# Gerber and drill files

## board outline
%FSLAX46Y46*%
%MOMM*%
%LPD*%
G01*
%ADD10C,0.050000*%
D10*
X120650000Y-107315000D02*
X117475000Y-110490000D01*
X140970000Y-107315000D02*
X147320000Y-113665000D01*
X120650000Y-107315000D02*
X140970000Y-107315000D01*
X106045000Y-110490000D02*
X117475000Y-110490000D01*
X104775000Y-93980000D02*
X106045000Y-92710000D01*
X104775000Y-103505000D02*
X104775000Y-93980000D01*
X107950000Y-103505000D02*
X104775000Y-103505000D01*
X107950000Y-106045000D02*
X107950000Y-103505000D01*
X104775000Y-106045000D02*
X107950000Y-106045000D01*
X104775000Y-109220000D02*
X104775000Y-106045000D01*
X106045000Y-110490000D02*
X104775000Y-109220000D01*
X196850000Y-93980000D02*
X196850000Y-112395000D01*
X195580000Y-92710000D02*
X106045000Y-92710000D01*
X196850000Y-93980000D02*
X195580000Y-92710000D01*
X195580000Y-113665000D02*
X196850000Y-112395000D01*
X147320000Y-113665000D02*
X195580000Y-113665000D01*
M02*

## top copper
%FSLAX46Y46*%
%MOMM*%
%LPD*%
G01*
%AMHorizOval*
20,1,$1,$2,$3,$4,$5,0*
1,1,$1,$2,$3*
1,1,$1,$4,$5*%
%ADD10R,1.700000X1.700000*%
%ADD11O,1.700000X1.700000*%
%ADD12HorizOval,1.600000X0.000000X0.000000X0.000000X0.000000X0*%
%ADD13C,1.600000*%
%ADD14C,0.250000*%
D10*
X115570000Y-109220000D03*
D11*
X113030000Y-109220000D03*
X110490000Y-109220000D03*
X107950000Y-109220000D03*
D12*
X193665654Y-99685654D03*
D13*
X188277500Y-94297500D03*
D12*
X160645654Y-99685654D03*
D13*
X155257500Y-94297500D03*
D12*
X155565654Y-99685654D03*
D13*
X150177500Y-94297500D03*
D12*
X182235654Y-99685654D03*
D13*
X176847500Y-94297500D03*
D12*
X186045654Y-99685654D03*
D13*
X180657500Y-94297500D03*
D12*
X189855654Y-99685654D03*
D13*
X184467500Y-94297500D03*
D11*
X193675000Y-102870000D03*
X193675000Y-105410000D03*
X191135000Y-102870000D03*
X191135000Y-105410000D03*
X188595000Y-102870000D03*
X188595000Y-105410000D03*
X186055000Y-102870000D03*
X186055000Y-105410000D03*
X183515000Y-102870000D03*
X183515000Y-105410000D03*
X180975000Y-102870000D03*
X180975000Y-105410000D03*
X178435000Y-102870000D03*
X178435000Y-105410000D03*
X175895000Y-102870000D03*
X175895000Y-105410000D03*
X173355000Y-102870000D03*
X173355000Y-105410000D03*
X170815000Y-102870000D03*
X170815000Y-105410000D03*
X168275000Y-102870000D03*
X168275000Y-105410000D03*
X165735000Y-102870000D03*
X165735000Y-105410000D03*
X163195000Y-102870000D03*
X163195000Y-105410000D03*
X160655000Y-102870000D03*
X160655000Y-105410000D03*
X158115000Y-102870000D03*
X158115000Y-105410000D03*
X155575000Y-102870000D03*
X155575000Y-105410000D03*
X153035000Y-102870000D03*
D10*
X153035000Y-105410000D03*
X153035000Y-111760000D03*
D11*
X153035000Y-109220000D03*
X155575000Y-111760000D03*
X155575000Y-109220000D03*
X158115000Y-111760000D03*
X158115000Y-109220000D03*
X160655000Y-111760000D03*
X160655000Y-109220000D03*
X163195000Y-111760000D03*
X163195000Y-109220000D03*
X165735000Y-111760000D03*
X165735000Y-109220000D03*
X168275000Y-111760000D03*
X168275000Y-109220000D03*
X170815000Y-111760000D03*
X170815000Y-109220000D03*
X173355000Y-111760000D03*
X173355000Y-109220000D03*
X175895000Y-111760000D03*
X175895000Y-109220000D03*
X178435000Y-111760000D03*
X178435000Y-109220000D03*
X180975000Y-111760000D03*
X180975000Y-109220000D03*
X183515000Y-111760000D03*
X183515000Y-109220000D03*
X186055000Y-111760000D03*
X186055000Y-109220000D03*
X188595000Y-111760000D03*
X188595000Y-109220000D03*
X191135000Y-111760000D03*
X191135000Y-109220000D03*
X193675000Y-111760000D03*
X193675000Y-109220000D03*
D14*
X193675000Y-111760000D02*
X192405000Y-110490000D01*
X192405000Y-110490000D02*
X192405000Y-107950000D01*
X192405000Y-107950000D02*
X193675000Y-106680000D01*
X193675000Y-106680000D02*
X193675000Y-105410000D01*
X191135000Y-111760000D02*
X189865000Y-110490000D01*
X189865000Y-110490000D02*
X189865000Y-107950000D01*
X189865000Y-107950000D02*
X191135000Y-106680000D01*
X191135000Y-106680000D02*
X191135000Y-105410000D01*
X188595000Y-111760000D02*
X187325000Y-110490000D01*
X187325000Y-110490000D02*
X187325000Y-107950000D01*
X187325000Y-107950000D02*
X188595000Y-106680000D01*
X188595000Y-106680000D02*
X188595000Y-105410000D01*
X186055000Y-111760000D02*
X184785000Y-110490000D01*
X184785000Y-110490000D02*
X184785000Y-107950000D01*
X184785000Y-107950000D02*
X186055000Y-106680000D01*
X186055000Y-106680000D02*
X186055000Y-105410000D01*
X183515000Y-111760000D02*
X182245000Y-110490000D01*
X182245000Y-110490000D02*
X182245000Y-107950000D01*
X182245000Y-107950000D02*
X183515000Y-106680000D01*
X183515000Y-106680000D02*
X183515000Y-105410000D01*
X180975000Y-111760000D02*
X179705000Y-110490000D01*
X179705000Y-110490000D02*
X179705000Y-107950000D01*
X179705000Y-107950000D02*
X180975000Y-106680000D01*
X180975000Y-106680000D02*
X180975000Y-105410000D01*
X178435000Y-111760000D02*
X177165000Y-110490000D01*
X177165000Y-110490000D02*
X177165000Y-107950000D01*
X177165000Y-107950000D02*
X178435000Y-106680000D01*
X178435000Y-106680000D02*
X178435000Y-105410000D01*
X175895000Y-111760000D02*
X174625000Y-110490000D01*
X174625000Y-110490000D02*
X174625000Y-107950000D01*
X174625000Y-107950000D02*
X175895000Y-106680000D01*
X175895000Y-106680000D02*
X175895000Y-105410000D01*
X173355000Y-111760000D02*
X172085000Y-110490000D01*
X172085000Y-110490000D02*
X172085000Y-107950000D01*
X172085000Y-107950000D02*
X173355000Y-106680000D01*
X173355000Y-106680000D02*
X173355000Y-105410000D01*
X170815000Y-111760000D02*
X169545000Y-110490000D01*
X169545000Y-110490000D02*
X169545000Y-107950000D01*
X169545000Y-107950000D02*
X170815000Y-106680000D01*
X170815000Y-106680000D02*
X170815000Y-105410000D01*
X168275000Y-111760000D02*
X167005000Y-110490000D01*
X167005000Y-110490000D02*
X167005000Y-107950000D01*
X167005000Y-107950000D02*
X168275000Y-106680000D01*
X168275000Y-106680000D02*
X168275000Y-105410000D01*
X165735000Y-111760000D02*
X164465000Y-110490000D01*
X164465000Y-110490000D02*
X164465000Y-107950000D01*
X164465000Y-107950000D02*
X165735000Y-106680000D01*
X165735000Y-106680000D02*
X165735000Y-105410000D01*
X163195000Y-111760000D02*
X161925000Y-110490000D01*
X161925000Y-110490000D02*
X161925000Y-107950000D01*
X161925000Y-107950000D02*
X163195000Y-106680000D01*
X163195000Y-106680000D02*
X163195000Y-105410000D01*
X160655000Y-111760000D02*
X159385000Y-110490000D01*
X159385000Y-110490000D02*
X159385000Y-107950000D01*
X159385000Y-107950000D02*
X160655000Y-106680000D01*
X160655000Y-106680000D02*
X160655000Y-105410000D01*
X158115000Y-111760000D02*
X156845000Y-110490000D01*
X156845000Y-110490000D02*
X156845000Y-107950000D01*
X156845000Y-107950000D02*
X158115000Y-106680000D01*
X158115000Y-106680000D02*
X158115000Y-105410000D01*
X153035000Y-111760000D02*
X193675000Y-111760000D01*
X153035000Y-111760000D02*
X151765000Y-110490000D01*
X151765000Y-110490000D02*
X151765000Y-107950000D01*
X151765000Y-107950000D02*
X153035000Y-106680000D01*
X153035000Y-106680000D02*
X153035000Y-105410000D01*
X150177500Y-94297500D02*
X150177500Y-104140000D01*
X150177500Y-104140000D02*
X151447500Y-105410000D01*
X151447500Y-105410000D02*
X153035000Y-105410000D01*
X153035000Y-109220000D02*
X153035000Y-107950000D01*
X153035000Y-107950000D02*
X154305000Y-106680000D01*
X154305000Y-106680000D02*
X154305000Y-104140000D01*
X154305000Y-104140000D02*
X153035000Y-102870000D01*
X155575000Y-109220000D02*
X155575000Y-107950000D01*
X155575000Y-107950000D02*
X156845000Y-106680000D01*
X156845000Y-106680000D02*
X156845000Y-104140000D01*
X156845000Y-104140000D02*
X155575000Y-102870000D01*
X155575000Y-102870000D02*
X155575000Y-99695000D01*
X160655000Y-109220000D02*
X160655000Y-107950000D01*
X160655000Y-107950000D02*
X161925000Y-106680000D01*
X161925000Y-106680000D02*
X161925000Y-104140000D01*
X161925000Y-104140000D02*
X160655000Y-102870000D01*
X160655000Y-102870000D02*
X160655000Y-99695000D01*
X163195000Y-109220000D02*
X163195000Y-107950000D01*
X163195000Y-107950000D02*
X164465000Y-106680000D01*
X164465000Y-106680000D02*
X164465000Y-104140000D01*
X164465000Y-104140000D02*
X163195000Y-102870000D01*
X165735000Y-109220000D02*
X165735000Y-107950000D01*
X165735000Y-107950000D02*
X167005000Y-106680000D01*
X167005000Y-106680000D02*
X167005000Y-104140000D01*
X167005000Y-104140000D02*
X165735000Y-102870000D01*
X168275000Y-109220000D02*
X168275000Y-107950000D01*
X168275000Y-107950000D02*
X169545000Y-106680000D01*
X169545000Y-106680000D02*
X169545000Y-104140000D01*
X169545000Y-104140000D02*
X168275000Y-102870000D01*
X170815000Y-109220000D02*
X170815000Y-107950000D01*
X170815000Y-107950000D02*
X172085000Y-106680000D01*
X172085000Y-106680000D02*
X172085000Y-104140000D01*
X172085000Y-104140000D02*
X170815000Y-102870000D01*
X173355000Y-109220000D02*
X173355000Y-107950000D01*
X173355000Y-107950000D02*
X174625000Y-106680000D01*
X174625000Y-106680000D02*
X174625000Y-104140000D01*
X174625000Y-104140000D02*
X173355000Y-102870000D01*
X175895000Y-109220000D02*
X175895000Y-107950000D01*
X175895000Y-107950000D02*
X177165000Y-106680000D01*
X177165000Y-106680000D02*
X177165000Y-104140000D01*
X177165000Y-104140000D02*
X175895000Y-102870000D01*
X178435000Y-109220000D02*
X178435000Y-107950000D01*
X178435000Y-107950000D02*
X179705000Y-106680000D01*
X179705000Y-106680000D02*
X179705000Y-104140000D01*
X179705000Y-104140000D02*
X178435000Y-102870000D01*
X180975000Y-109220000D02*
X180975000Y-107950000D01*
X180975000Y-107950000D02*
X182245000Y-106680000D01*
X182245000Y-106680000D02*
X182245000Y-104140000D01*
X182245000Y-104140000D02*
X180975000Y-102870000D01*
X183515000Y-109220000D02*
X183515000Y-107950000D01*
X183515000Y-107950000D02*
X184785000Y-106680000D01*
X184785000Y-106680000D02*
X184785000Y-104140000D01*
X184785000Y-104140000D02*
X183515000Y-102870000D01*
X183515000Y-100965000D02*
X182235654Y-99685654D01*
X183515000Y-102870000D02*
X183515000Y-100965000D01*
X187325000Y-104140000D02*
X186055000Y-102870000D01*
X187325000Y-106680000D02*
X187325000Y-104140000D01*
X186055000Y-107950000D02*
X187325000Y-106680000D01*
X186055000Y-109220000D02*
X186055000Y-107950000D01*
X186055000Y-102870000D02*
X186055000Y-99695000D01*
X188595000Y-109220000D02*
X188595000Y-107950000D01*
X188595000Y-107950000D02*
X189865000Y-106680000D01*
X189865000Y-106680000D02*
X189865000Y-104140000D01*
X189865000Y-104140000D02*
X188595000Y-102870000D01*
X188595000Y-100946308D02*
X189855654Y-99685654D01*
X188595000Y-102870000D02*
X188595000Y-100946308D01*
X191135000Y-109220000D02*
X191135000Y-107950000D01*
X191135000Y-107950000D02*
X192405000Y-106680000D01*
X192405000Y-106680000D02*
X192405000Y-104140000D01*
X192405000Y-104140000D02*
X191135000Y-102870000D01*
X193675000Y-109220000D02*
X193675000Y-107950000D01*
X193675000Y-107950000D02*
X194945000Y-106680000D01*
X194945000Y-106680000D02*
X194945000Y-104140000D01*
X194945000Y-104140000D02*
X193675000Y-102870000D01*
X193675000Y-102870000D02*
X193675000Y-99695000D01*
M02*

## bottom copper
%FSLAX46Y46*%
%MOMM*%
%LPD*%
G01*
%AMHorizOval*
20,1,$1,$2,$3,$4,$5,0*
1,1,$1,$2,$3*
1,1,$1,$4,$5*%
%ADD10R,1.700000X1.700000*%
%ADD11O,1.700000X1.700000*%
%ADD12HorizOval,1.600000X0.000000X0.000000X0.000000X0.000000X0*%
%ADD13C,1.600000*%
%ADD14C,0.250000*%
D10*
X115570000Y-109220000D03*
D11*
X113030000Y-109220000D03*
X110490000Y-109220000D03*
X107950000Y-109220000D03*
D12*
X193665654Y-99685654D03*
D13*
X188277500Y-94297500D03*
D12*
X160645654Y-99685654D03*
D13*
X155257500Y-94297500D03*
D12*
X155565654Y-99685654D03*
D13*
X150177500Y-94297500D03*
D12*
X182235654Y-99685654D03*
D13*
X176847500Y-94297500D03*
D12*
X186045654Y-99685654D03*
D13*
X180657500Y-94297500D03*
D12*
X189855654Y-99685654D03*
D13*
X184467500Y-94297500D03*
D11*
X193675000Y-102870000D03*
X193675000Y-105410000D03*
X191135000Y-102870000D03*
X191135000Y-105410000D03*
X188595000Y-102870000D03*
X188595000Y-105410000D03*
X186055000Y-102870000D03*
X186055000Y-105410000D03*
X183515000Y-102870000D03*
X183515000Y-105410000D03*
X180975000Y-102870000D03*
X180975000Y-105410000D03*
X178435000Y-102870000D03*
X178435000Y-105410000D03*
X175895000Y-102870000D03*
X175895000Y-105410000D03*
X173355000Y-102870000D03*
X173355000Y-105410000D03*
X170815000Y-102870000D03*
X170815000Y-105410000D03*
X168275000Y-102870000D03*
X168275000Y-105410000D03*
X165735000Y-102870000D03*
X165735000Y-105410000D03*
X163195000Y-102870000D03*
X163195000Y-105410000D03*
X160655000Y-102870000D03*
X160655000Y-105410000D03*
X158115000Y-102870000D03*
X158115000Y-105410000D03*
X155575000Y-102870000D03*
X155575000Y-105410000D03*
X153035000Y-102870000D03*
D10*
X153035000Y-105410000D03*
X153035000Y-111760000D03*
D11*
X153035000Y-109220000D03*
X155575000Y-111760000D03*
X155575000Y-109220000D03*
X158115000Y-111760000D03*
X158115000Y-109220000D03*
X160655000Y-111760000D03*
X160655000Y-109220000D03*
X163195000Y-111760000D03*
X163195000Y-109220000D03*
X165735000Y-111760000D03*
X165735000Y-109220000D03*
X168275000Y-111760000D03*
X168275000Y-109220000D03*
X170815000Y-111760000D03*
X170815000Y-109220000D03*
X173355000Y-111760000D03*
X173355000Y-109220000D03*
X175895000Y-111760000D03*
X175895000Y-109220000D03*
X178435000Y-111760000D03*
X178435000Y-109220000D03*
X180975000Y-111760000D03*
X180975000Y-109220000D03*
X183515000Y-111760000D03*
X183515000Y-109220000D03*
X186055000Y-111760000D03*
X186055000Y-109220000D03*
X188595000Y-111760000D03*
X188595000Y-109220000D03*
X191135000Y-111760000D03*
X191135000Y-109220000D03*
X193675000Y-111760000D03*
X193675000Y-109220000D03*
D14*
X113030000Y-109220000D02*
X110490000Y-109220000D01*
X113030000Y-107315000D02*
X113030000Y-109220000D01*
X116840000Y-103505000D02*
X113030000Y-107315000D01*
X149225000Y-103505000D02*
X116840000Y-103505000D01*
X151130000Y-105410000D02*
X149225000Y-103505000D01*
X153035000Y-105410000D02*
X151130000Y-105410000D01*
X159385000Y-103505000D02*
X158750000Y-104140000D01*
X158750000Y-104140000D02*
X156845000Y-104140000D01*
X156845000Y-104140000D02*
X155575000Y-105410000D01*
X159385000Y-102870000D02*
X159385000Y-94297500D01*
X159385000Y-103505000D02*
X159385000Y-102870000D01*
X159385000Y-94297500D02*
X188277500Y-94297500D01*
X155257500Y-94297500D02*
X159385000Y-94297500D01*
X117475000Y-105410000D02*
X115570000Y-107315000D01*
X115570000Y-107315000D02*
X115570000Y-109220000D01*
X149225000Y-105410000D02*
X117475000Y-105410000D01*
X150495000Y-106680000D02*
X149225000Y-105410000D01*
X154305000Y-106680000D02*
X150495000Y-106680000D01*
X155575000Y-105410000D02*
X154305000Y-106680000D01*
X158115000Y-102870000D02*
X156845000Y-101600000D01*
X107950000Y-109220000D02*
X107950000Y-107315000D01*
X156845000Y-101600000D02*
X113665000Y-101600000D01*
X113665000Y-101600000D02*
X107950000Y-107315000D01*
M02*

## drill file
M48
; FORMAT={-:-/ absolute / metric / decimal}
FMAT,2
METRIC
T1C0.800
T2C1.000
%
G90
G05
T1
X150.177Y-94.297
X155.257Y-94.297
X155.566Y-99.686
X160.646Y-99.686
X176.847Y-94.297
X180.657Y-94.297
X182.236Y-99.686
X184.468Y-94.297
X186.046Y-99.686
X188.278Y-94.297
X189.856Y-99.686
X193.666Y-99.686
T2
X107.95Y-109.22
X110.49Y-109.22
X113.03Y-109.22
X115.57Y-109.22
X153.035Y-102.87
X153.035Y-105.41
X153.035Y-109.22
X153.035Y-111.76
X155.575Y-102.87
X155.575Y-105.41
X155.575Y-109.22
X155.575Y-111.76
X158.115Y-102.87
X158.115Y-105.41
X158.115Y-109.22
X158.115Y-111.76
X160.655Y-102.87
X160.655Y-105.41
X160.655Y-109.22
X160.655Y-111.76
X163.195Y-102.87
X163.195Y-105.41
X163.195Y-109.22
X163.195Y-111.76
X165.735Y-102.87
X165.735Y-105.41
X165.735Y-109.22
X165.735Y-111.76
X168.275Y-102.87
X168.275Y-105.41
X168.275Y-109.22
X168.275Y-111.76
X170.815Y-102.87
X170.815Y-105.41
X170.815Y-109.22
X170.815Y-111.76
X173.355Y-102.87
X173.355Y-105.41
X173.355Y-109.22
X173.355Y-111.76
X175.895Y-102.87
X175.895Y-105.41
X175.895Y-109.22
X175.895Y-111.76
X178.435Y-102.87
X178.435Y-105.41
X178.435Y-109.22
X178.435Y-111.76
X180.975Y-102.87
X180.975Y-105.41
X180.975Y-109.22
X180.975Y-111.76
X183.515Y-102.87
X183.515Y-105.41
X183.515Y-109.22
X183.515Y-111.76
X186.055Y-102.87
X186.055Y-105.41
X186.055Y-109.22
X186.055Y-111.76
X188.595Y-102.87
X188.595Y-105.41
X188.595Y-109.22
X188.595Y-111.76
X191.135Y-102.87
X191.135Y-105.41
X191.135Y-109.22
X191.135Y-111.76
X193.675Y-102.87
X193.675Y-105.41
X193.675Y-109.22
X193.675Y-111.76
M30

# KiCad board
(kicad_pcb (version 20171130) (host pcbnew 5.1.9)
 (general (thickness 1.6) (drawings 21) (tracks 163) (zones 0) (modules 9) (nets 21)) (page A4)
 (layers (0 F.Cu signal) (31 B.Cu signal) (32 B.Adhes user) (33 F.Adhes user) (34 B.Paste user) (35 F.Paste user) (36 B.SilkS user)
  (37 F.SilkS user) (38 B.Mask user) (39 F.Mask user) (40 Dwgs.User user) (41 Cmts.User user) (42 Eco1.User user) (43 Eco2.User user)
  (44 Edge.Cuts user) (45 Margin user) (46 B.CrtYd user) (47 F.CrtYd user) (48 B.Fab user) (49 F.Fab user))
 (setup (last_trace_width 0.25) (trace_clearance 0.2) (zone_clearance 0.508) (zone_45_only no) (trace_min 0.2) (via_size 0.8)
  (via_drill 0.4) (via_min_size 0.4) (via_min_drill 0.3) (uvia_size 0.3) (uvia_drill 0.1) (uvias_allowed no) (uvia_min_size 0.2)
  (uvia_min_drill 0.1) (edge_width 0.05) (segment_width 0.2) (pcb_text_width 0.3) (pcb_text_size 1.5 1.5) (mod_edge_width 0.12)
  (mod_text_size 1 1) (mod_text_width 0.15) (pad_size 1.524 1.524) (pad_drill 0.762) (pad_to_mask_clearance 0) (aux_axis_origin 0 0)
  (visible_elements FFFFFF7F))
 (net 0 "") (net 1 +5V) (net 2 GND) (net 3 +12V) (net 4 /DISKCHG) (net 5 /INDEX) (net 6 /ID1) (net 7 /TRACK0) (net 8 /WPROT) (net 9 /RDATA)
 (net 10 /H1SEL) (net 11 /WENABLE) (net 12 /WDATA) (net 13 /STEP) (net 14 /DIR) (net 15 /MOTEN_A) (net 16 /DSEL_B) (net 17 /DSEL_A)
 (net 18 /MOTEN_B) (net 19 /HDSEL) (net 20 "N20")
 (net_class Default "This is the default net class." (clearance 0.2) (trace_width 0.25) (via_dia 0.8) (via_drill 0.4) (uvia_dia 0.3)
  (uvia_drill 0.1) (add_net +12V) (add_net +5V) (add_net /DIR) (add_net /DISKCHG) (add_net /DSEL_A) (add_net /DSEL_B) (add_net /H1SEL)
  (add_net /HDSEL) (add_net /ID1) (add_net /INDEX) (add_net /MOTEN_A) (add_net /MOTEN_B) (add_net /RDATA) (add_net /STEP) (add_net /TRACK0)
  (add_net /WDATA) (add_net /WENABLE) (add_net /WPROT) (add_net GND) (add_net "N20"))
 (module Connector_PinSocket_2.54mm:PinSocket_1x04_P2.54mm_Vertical (layer B.Cu) (at 115.57 109.22 90)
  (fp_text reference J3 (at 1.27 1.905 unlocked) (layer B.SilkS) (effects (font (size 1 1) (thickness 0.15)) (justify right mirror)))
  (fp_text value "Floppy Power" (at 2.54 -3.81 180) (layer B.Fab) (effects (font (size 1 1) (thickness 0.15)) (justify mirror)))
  (pad 1 thru_hole rect (at 0 0 90) (size 1.7 1.7) (drill 1) (layers *.Cu *.Mask) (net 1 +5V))
  (pad 2 thru_hole oval (at 0 -2.54 90) (size 1.7 1.7) (drill 1) (layers *.Cu *.Mask) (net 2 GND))
  (pad 3 thru_hole oval (at 0 -5.08 90) (size 1.7 1.7) (drill 1) (layers *.Cu *.Mask) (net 2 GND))
  (pad 4 thru_hole oval (at 0 -7.62 90) (size 1.7 1.7) (drill 1) (layers *.Cu *.Mask) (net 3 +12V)))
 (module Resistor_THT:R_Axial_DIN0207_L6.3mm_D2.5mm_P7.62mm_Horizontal (layer F.Cu) (at 188.2775 94.2975 315)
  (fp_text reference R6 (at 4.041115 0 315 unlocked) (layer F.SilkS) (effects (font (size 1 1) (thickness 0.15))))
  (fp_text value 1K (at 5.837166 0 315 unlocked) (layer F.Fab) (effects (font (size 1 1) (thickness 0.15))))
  (pad 2 thru_hole oval (at 7.62 0 315) (size 1.6 1.6) (drill 0.8) (layers *.Cu *.Mask) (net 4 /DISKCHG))
  (pad 1 thru_hole circle (at 0 0 315) (size 1.6 1.6) (drill 0.8) (layers *.Cu *.Mask) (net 1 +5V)))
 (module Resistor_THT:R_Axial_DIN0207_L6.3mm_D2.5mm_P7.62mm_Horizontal (layer F.Cu) (at 155.2575 94.2975 315)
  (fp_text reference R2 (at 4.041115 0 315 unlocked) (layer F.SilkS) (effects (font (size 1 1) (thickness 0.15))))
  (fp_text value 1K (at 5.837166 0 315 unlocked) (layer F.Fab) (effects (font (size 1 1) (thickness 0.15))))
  (pad 2 thru_hole oval (at 7.62 0 315) (size 1.6 1.6) (drill 0.8) (layers *.Cu *.Mask) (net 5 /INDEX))
  (pad 1 thru_hole circle (at 0 0 315) (size 1.6 1.6) (drill 0.8) (layers *.Cu *.Mask) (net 1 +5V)))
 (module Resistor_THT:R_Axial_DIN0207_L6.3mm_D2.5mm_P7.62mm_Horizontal (layer F.Cu) (at 150.1775 94.2975 315)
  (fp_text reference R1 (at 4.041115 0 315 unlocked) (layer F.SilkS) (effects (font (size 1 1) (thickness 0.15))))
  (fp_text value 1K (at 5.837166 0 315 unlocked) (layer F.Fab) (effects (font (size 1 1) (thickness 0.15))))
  (pad 2 thru_hole oval (at 7.62 0 315) (size 1.6 1.6) (drill 0.8) (layers *.Cu *.Mask) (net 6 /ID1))
  (pad 1 thru_hole circle (at 0 0 315) (size 1.6 1.6) (drill 0.8) (layers *.Cu *.Mask) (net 2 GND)))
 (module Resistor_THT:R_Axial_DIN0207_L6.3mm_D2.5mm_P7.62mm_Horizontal (layer F.Cu) (at 176.8475 94.2975 315)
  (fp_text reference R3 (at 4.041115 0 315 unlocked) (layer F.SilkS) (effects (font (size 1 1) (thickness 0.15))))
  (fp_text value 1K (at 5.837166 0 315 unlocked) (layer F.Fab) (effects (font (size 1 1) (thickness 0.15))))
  (pad 2 thru_hole oval (at 7.62 0 315) (size 1.6 1.6) (drill 0.8) (layers *.Cu *.Mask) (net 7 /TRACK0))
  (pad 1 thru_hole circle (at 0 0 315) (size 1.6 1.6) (drill 0.8) (layers *.Cu *.Mask) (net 1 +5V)))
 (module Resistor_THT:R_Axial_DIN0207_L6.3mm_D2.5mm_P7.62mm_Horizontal (layer F.Cu) (at 180.6575 94.2975 315)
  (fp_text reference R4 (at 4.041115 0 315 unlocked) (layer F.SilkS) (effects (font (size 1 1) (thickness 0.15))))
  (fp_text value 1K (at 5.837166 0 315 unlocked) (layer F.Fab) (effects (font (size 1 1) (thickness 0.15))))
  (pad 2 thru_hole oval (at 7.62 0 315) (size 1.6 1.6) (drill 0.8) (layers *.Cu *.Mask) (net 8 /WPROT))
  (pad 1 thru_hole circle (at 0 0 315) (size 1.6 1.6) (drill 0.8) (layers *.Cu *.Mask) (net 1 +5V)))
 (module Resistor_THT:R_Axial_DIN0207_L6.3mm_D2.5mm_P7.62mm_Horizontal (layer F.Cu) (at 184.4675 94.2975 315)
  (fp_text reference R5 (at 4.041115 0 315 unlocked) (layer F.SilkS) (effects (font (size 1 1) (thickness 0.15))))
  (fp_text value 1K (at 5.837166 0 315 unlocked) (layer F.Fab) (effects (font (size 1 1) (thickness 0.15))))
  (pad 2 thru_hole oval (at 7.62 0 315) (size 1.6 1.6) (drill 0.8) (layers *.Cu *.Mask) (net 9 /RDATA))
  (pad 1 thru_hole circle (at 0 0 315) (size 1.6 1.6) (drill 0.8) (layers *.Cu *.Mask) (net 1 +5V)))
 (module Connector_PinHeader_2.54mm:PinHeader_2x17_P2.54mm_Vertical (layer F.Cu) (at 153.035 105.41 90)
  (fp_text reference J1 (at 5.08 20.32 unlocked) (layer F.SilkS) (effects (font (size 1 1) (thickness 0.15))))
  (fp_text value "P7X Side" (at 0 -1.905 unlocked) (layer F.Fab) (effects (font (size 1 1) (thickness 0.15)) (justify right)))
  (pad 34 thru_hole oval (at 2.54 40.64 90) (size 1.7 1.7) (drill 1) (layers *.Cu *.Mask) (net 4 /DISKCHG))
  (pad 33 thru_hole oval (at 0 40.64 90) (size 1.7 1.7) (drill 1) (layers *.Cu *.Mask) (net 2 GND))
  (pad 32 thru_hole oval (at 2.54 38.1 90) (size 1.7 1.7) (drill 1) (layers *.Cu *.Mask) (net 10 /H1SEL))
  (pad 31 thru_hole oval (at 0 38.1 90) (size 1.7 1.7) (drill 1) (layers *.Cu *.Mask) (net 2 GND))
  (pad 30 thru_hole oval (at 2.54 35.56 90) (size 1.7 1.7) (drill 1) (layers *.Cu *.Mask) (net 9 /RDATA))
  (pad 29 thru_hole oval (at 0 35.56 90) (size 1.7 1.7) (drill 1) (layers *.Cu *.Mask) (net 2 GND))
  (pad 28 thru_hole oval (at 2.54 33.02 90) (size 1.7 1.7) (drill 1) (layers *.Cu *.Mask) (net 8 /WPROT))
  (pad 27 thru_hole oval (at 0 33.02 90) (size 1.7 1.7) (drill 1) (layers *.Cu *.Mask) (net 2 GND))
  (pad 26 thru_hole oval (at 2.54 30.48 90) (size 1.7 1.7) (drill 1) (layers *.Cu *.Mask) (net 7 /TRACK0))
  (pad 25 thru_hole oval (at 0 30.48 90) (size 1.7 1.7) (drill 1) (layers *.Cu *.Mask) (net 2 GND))
  (pad 24 thru_hole oval (at 2.54 27.94 90) (size 1.7 1.7) (drill 1) (layers *.Cu *.Mask) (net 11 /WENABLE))
  (pad 23 thru_hole oval (at 0 27.94 90) (size 1.7 1.7) (drill 1) (layers *.Cu *.Mask) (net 2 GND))
  (pad 22 thru_hole oval (at 2.54 25.4 90) (size 1.7 1.7) (drill 1) (layers *.Cu *.Mask) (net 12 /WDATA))
  (pad 21 thru_hole oval (at 0 25.4 90) (size 1.7 1.7) (drill 1) (layers *.Cu *.Mask) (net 2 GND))
  (pad 20 thru_hole oval (at 2.54 22.86 90) (size 1.7 1.7) (drill 1) (layers *.Cu *.Mask) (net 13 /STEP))
  (pad 19 thru_hole oval (at 0 22.86 90) (size 1.7 1.7) (drill 1) (layers *.Cu *.Mask) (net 2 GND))
  (pad 18 thru_hole oval (at 2.54 20.32 90) (size 1.7 1.7) (drill 1) (layers *.Cu *.Mask) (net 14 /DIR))
  (pad 17 thru_hole oval (at 0 20.32 90) (size 1.7 1.7) (drill 1) (layers *.Cu *.Mask) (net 2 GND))
  (pad 16 thru_hole oval (at 2.54 17.78 90) (size 1.7 1.7) (drill 1) (layers *.Cu *.Mask) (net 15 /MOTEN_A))
  (pad 15 thru_hole oval (at 0 17.78 90) (size 1.7 1.7) (drill 1) (layers *.Cu *.Mask) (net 2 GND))
  (pad 14 thru_hole oval (at 2.54 15.24 90) (size 1.7 1.7) (drill 1) (layers *.Cu *.Mask) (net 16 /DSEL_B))
  (pad 13 thru_hole oval (at 0 15.24 90) (size 1.7 1.7) (drill 1) (layers *.Cu *.Mask) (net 2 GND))
  (pad 12 thru_hole oval (at 2.54 12.7 90) (size 1.7 1.7) (drill 1) (layers *.Cu *.Mask) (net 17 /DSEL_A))
  (pad 11 thru_hole oval (at 0 12.7 90) (size 1.7 1.7) (drill 1) (layers *.Cu *.Mask) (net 2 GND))
  (pad 10 thru_hole oval (at 2.54 10.16 90) (size 1.7 1.7) (drill 1) (layers *.Cu *.Mask) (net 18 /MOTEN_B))
  (pad 9 thru_hole oval (at 0 10.16 90) (size 1.7 1.7) (drill 1) (layers *.Cu *.Mask) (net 2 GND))
  (pad 8 thru_hole oval (at 2.54 7.62 90) (size 1.7 1.7) (drill 1) (layers *.Cu *.Mask) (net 5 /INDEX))
  (pad 7 thru_hole oval (at 0 7.62 90) (size 1.7 1.7) (drill 1) (layers *.Cu *.Mask) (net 2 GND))
  (pad 6 thru_hole oval (at 2.54 5.08 90) (size 1.7 1.7) (drill 1) (layers *.Cu *.Mask) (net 3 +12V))
  (pad 5 thru_hole oval (at 0 5.08 90) (size 1.7 1.7) (drill 1) (layers *.Cu *.Mask) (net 2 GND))
  (pad 4 thru_hole oval (at 2.54 2.54 90) (size 1.7 1.7) (drill 1) (layers *.Cu *.Mask) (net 6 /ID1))
  (pad 3 thru_hole oval (at 0 2.54 90) (size 1.7 1.7) (drill 1) (layers *.Cu *.Mask) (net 1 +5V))
  (pad 2 thru_hole oval (at 2.54 0 90) (size 1.7 1.7) (drill 1) (layers *.Cu *.Mask) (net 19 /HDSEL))
  (pad 1 thru_hole rect (at 0 0 90) (size 1.7 1.7) (drill 1) (layers *.Cu *.Mask) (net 2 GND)))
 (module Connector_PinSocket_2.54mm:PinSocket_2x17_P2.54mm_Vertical (layer B.Cu) (at 153.035 111.76 270)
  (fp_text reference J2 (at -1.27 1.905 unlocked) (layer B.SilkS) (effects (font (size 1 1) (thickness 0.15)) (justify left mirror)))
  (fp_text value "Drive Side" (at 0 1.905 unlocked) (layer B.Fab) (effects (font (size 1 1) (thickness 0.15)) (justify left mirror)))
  (pad 1 thru_hole rect (at 0 0 270) (size 1.7 1.7) (drill 1) (layers *.Cu *.Mask) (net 2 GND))
  (pad 2 thru_hole oval (at -2.54 0 270) (size 1.7 1.7) (drill 1) (layers *.Cu *.Mask) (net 19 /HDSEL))
  (pad 3 thru_hole oval (at 0 -2.54 270) (size 1.7 1.7) (drill 1) (layers *.Cu *.Mask) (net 2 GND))
  (pad 4 thru_hole oval (at -2.54 -2.54 270) (size 1.7 1.7) (drill 1) (layers *.Cu *.Mask) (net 6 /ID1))
  (pad 5 thru_hole oval (at 0 -5.08 270) (size 1.7 1.7) (drill 1) (layers *.Cu *.Mask) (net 2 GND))
  (pad 6 thru_hole oval (at -2.54 -5.08 270) (size 1.7 1.7) (drill 1) (layers *.Cu *.Mask) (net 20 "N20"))
  (pad 7 thru_hole oval (at 0 -7.62 270) (size 1.7 1.7) (drill 1) (layers *.Cu *.Mask) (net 2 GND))
  (pad 8 thru_hole oval (at -2.54 -7.62 270) (size 1.7 1.7) (drill 1) (layers *.Cu *.Mask) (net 5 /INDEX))
  (pad 9 thru_hole oval (at 0 -10.16 270) (size 1.7 1.7) (drill 1) (layers *.Cu *.Mask) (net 2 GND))
  (pad 10 thru_hole oval (at -2.54 -10.16 270) (size 1.7 1.7) (drill 1) (layers *.Cu *.Mask) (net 18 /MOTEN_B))
  (pad 11 thru_hole oval (at 0 -12.7 270) (size 1.7 1.7) (drill 1) (layers *.Cu *.Mask) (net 2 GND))
  (pad 12 thru_hole oval (at -2.54 -12.7 270) (size 1.7 1.7) (drill 1) (layers *.Cu *.Mask) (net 17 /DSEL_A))
  (pad 13 thru_hole oval (at 0 -15.24 270) (size 1.7 1.7) (drill 1) (layers *.Cu *.Mask) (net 2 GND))
  (pad 14 thru_hole oval (at -2.54 -15.24 270) (size 1.7 1.7) (drill 1) (layers *.Cu *.Mask) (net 16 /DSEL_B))
  (pad 15 thru_hole oval (at 0 -17.78 270) (size 1.7 1.7) (drill 1) (layers *.Cu *.Mask) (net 2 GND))
  (pad 16 thru_hole oval (at -2.54 -17.78 270) (size 1.7 1.7) (drill 1) (layers *.Cu *.Mask) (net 15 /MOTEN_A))
  (pad 17 thru_hole oval (at 0 -20.32 270) (size 1.7 1.7) (drill 1) (layers *.Cu *.Mask) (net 2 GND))
  (pad 18 thru_hole oval (at -2.54 -20.32 270) (size 1.7 1.7) (drill 1) (layers *.Cu *.Mask) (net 14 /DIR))
  (pad 19 thru_hole oval (at 0 -22.86 270) (size 1.7 1.7) (drill 1) (layers *.Cu *.Mask) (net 2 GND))
  (pad 20 thru_hole oval (at -2.54 -22.86 270) (size 1.7 1.7) (drill 1) (layers *.Cu *.Mask) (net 13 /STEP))
  (pad 21 thru_hole oval (at 0 -25.4 270) (size 1.7 1.7) (drill 1) (layers *.Cu *.Mask) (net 2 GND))
  (pad 22 thru_hole oval (at -2.54 -25.4 270) (size 1.7 1.7) (drill 1) (layers *.Cu *.Mask) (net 12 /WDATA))
  (pad 23 thru_hole oval (at 0 -27.94 270) (size 1.7 1.7) (drill 1) (layers *.Cu *.Mask) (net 2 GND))
  (pad 24 thru_hole oval (at -2.54 -27.94 270) (size 1.7 1.7) (drill 1) (layers *.Cu *.Mask) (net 11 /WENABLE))
  (pad 25 thru_hole oval (at 0 -30.48 270) (size 1.7 1.7) (drill 1) (layers *.Cu *.Mask) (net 2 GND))
  (pad 26 thru_hole oval (at -2.54 -30.48 270) (size 1.7 1.7) (drill 1) (layers *.Cu *.Mask) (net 7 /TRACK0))
  (pad 27 thru_hole oval (at 0 -33.02 270) (size 1.7 1.7) (drill 1) (layers *.Cu *.Mask) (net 2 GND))
  (pad 28 thru_hole oval (at -2.54 -33.02 270) (size 1.7 1.7) (drill 1) (layers *.Cu *.Mask) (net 8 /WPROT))
  (pad 29 thru_hole oval (at 0 -35.56 270) (size 1.7 1.7) (drill 1) (layers *.Cu *.Mask) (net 2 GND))
  (pad 30 thru_hole oval (at -2.54 -35.56 270) (size 1.7 1.7) (drill 1) (layers *.Cu *.Mask) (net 9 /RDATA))
  (pad 31 thru_hole oval (at 0 -38.1 270) (size 1.7 1.7) (drill 1) (layers *.Cu *.Mask) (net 2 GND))
  (pad 32 thru_hole oval (at -2.54 -38.1 270) (size 1.7 1.7) (drill 1) (layers *.Cu *.Mask) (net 10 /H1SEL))
  (pad 33 thru_hole oval (at 0 -40.64 270) (size 1.7 1.7) (drill 1) (layers *.Cu *.Mask) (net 2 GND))
  (pad 34 thru_hole oval (at -2.54 -40.64 270) (size 1.7 1.7) (drill 1) (layers *.Cu *.Mask) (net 4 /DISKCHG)))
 (gr_line (start 120.65 107.315) (end 117.475 110.49) (layer Edge.Cuts) (width 0.05))
 (gr_line (start 140.97 107.315) (end 147.32 113.665) (layer Edge.Cuts) (width 0.05))
 (gr_line (start 120.65 107.315) (end 140.97 107.315) (layer Edge.Cuts) (width 0.05))
 (gr_line (start 106.045 110.49) (end 117.475 110.49) (layer Edge.Cuts) (width 0.05))
 (gr_line (start 104.775 93.98) (end 106.045 92.71) (layer Edge.Cuts) (width 0.05))
 (gr_line (start 104.775 103.505) (end 104.775 93.98) (layer Edge.Cuts) (width 0.05))
 (gr_line (start 107.95 103.505) (end 104.775 103.505) (layer Edge.Cuts) (width 0.05))
 (gr_line (start 107.95 106.045) (end 107.95 103.505) (layer Edge.Cuts) (width 0.05))
 (gr_line (start 104.775 106.045) (end 107.95 106.045) (layer Edge.Cuts) (width 0.05))
 (gr_line (start 104.775 109.22) (end 104.775 106.045) (layer Edge.Cuts) (width 0.05))
 (gr_line (start 106.045 110.49) (end 104.775 109.22) (layer Edge.Cuts) (width 0.05))
 (gr_line (start 196.85 93.98) (end 196.85 112.395) (layer Edge.Cuts) (width 0.05))
 (gr_line (start 195.58 92.71) (end 106.045 92.71) (layer Edge.Cuts) (width 0.05))
 (gr_line (start 196.85 93.98) (end 195.58 92.71) (layer Edge.Cuts) (width 0.05))
 (gr_line (start 195.58 113.665) (end 196.85 112.395) (layer Edge.Cuts) (width 0.05))
 (gr_line (start 147.32 113.665) (end 195.58 113.665) (layer Edge.Cuts) (width 0.05))
 (segment (start 193.675 111.76) (end 192.405 110.49) (width 0.25) (layer F.Cu) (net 2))
 (segment (start 192.405 110.49) (end 192.405 107.95) (width 0.25) (layer F.Cu) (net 2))
 (segment (start 192.405 107.95) (end 193.675 106.68) (width 0.25) (layer F.Cu) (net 2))
 (segment (start 193.675 106.68) (end 193.675 105.41) (width 0.25) (layer F.Cu) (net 2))
 (segment (start 191.135 111.76) (end 189.865 110.49) (width 0.25) (layer F.Cu) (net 2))
 (segment (start 189.865 110.49) (end 189.865 107.95) (width 0.25) (layer F.Cu) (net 2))
 (segment (start 189.865 107.95) (end 191.135 106.68) (width 0.25) (layer F.Cu) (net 2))
 (segment (start 191.135 106.68) (end 191.135 105.41) (width 0.25) (layer F.Cu) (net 2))
 (segment (start 188.595 111.76) (end 187.325 110.49) (width 0.25) (layer F.Cu) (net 2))
 (segment (start 187.325 110.49) (end 187.325 107.95) (width 0.25) (layer F.Cu) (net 2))
 (segment (start 187.325 107.95) (end 188.595 106.68) (width 0.25) (layer F.Cu) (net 2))
 (segment (start 188.595 106.68) (end 188.595 105.41) (width 0.25) (layer F.Cu) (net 2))
 (segment (start 186.055 111.76) (end 184.785 110.49) (width 0.25) (layer F.Cu) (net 2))
 (segment (start 184.785 110.49) (end 184.785 107.95) (width 0.25) (layer F.Cu) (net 2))
 (segment (start 184.785 107.95) (end 186.055 106.68) (width 0.25) (layer F.Cu) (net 2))
 (segment (start 186.055 106.68) (end 186.055 105.41) (width 0.25) (layer F.Cu) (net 2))
 (segment (start 183.515 111.76) (end 182.245 110.49) (width 0.25) (layer F.Cu) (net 2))
 (segment (start 182.245 110.49) (end 182.245 107.95) (width 0.25) (layer F.Cu) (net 2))
 (segment (start 182.245 107.95) (end 183.515 106.68) (width 0.25) (layer F.Cu) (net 2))
 (segment (start 183.515 106.68) (end 183.515 105.41) (width 0.25) (layer F.Cu) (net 2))
 (segment (start 180.975 111.76) (end 179.705 110.49) (width 0.25) (layer F.Cu) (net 2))
 (segment (start 179.705 110.49) (end 179.705 107.95) (width 0.25) (layer F.Cu) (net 2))
 (segment (start 179.705 107.95) (end 180.975 106.68) (width 0.25) (layer F.Cu) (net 2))
 (segment (start 180.975 106.68) (end 180.975 105.41) (width 0.25) (layer F.Cu) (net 2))
 (segment (start 178.435 111.76) (end 177.165 110.49) (width 0.25) (layer F.Cu) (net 2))
 (segment (start 177.165 110.49) (end 177.165 107.95) (width 0.25) (layer F.Cu) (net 2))
 (segment (start 177.165 107.95) (end 178.435 106.68) (width 0.25) (layer F.Cu) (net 2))
 (segment (start 178.435 106.68) (end 178.435 105.41) (width 0.25) (layer F.Cu) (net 2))
 (segment (start 175.895 111.76) (end 174.625 110.49) (width 0.25) (layer F.Cu) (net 2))
 (segment (start 174.625 110.49) (end 174.625 107.95) (width 0.25) (layer F.Cu) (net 2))
 (segment (start 174.625 107.95) (end 175.895 106.68) (width 0.25) (layer F.Cu) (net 2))
 (segment (start 175.895 106.68) (end 175.895 105.41) (width 0.25) (layer F.Cu) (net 2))
 (segment (start 173.355 111.76) (end 172.085 110.49) (width 0.25) (layer F.Cu) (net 2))
 (segment (start 172.085 110.49) (end 172.085 107.95) (width 0.25) (layer F.Cu) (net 2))
 (segment (start 172.085 107.95) (end 173.355 106.68) (width 0.25) (layer F.Cu) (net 2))
 (segment (start 173.355 106.68) (end 173.355 105.41) (width 0.25) (layer F.Cu) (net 2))
 (segment (start 170.815 111.76) (end 169.545 110.49) (width 0.25) (layer F.Cu) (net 2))
 (segment (start 169.545 110.49) (end 169.545 107.95) (width 0.25) (layer F.Cu) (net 2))
 (segment (start 169.545 107.95) (end 170.815 106.68) (width 0.25) (layer F.Cu) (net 2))
 (segment (start 170.815 106.68) (end 170.815 105.41) (width 0.25) (layer F.Cu) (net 2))
 (segment (start 168.275 111.76) (end 167.005 110.49) (width 0.25) (layer F.Cu) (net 2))
 (segment (start 167.005 110.49) (end 167.005 107.95) (width 0.25) (layer F.Cu) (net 2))
 (segment (start 167.005 107.95) (end 168.275 106.68) (width 0.25) (layer F.Cu) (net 2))
 (segment (start 168.275 106.68) (end 168.275 105.41) (width 0.25) (layer F.Cu) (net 2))
 (segment (start 165.735 111.76) (end 164.465 110.49) (width 0.25) (layer F.Cu) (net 2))
 (segment (start 164.465 110.49) (end 164.465 107.95) (width 0.25) (layer F.Cu) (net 2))
 (segment (start 164.465 107.95) (end 165.735 106.68) (width 0.25) (layer F.Cu) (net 2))
 (segment (start 165.735 106.68) (end 165.735 105.41) (width 0.25) (layer F.Cu) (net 2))
 (segment (start 163.195 111.76) (end 161.925 110.49) (width 0.25) (layer F.Cu) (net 2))
 (segment (start 161.925 110.49) (end 161.925 107.95) (width 0.25) (layer F.Cu) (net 2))
 (segment (start 161.925 107.95) (end 163.195 106.68) (width 0.25) (layer F.Cu) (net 2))
 (segment (start 163.195 106.68) (end 163.195 105.41) (width 0.25) (layer F.Cu) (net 2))
 (segment (start 160.655 111.76) (end 159.385 110.49) (width 0.25) (layer F.Cu) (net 2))
 (segment (start 159.385 110.49) (end 159.385 107.95) (width 0.25) (layer F.Cu) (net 2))
 (segment (start 159.385 107.95) (end 160.655 106.68) (width 0.25) (layer F.Cu) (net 2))
 (segment (start 160.655 106.68) (end 160.655 105.41) (width 0.25) (layer F.Cu) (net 2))
 (segment (start 158.115 111.76) (end 156.845 110.49) (width 0.25) (layer F.Cu) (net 2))
 (segment (start 156.845 110.49) (end 156.845 107.95) (width 0.25) (layer F.Cu) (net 2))
 (segment (start 156.845 107.95) (end 158.115 106.68) (width 0.25) (layer F.Cu) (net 2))
 (segment (start 158.115 106.68) (end 158.115 105.41) (width 0.25) (layer F.Cu) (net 2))
 (segment (start 153.035 111.76) (end 193.675 111.76) (width 0.25) (layer F.Cu) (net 2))
 (segment (start 153.035 111.76) (end 151.765 110.49) (width 0.25) (layer F.Cu) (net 2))
 (segment (start 151.765 110.49) (end 151.765 107.95) (width 0.25) (layer F.Cu) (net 2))
 (segment (start 151.765 107.95) (end 153.035 106.68) (width 0.25) (layer F.Cu) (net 2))
 (segment (start 153.035 106.68) (end 153.035 105.41) (width 0.25) (layer F.Cu) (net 2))
 (segment (start 113.03 109.22) (end 110.49 109.22) (width 0.25) (layer B.Cu) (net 2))
 (segment (start 150.1775 94.2975) (end 150.1775 104.14) (width 0.25) (layer F.Cu) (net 2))
 (segment (start 150.1775 104.14) (end 151.4475 105.41) (width 0.25) (layer F.Cu) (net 2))
 (segment (start 151.4475 105.41) (end 153.035 105.41) (width 0.25) (layer F.Cu) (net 2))
 (segment (start 113.03 107.315) (end 113.03 109.22) (width 0.25) (layer B.Cu) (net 2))
 (segment (start 116.84 103.505) (end 113.03 107.315) (width 0.25) (layer B.Cu) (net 2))
 (segment (start 149.225 103.505) (end 116.84 103.505) (width 0.25) (layer B.Cu) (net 2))
 (segment (start 151.13 105.41) (end 149.225 103.505) (width 0.25) (layer B.Cu) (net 2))
 (segment (start 153.035 105.41) (end 151.13 105.41) (width 0.25) (layer B.Cu) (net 2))
 (segment (start 153.035 109.22) (end 153.035 107.95) (width 0.25) (layer F.Cu) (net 19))
 (segment (start 153.035 107.95) (end 154.305 106.68) (width 0.25) (layer F.Cu) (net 19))
 (segment (start 154.305 106.68) (end 154.305 104.14) (width 0.25) (layer F.Cu) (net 19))
 (segment (start 154.305 104.14) (end 153.035 102.87) (width 0.25) (layer F.Cu) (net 19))
 (segment (start 159.385 103.505) (end 158.75 104.14) (width 0.25) (layer B.Cu) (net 1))
 (segment (start 158.75 104.14) (end 156.845 104.14) (width 0.25) (layer B.Cu) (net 1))
 (segment (start 156.845 104.14) (end 155.575 105.41) (width 0.25) (layer B.Cu) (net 1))
 (segment (start 159.385 102.87) (end 159.385 94.2975) (width 0.25) (layer B.Cu) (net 1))
 (segment (start 159.385 103.505) (end 159.385 102.87) (width 0.25) (layer B.Cu) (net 1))
 (segment (start 159.385 94.2975) (end 188.2775 94.2975) (width 0.25) (layer B.Cu) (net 1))
 (segment (start 155.2575 94.2975) (end 159.385 94.2975) (width 0.25) (layer B.Cu) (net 1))
 (segment (start 117.475 105.41) (end 115.57 107.315) (width 0.25) (layer B.Cu) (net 1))
 (segment (start 115.57 107.315) (end 115.57 109.22) (width 0.25) (layer B.Cu) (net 1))
 (segment (start 149.225 105.41) (end 117.475 105.41) (width 0.25) (layer B.Cu) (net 1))
 (segment (start 150.495 106.68) (end 149.225 105.41) (width 0.25) (layer B.Cu) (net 1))
 (segment (start 154.305 106.68) (end 150.495 106.68) (width 0.25) (layer B.Cu) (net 1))
 (segment (start 155.575 105.41) (end 154.305 106.68) (width 0.25) (layer B.Cu) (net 1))
 (segment (start 155.575 109.22) (end 155.575 107.95) (width 0.25) (layer F.Cu) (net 6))
 (segment (start 155.575 107.95) (end 156.845 106.68) (width 0.25) (layer F.Cu) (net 6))
 (segment (start 156.845 106.68) (end 156.845 104.14) (width 0.25) (layer F.Cu) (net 6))
 (segment (start 156.845 104.14) (end 155.575 102.87) (width 0.25) (layer F.Cu) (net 6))
 (segment (start 155.575 102.87) (end 155.575 99.695) (width 0.25) (layer F.Cu) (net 6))
 (segment (start 158.115 102.87) (end 156.845 101.6) (width 0.25) (layer B.Cu) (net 3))
 (segment (start 107.95 109.22) (end 107.95 107.315) (width 0.25) (layer B.Cu) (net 3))
 (segment (start 156.845 101.6) (end 113.665 101.6) (width 0.25) (layer B.Cu) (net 3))
 (segment (start 113.665 101.6) (end 107.95 107.315) (width 0.25) (layer B.Cu) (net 3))
 (segment (start 160.655 109.22) (end 160.655 107.95) (width 0.25) (layer F.Cu) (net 5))
 (segment (start 160.655 107.95) (end 161.925 106.68) (width 0.25) (layer F.Cu) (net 5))
 (segment (start 161.925 106.68) (end 161.925 104.14) (width 0.25) (layer F.Cu) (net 5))
 (segment (start 161.925 104.14) (end 160.655 102.87) (width 0.25) (layer F.Cu) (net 5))
 (segment (start 160.655 102.87) (end 160.655 99.695) (width 0.25) (layer F.Cu) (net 5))
 (segment (start 163.195 109.22) (end 163.195 107.95) (width 0.25) (layer F.Cu) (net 18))
 (segment (start 163.195 107.95) (end 164.465 106.68) (width 0.25) (layer F.Cu) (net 18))
 (segment (start 164.465 106.68) (end 164.465 104.14) (width 0.25) (layer F.Cu) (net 18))
 (segment (start 164.465 104.14) (end 163.195 102.87) (width 0.25) (layer F.Cu) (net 18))
 (segment (start 165.735 109.22) (end 165.735 107.95) (width 0.25) (layer F.Cu) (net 17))
 (segment (start 165.735 107.95) (end 167.005 106.68) (width 0.25) (layer F.Cu) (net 17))
 (segment (start 167.005 106.68) (end 167.005 104.14) (width 0.25) (layer F.Cu) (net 17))
 (segment (start 167.005 104.14) (end 165.735 102.87) (width 0.25) (layer F.Cu) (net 17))
 (segment (start 168.275 109.22) (end 168.275 107.95) (width 0.25) (layer F.Cu) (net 16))
 (segment (start 168.275 107.95) (end 169.545 106.68) (width 0.25) (layer F.Cu) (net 16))
 (segment (start 169.545 106.68) (end 169.545 104.14) (width 0.25) (layer F.Cu) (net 16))
 (segment (start 169.545 104.14) (end 168.275 102.87) (width 0.25) (layer F.Cu) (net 16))
 (segment (start 170.815 109.22) (end 170.815 107.95) (width 0.25) (layer F.Cu) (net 15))
 (segment (start 170.815 107.95) (end 172.085 106.68) (width 0.25) (layer F.Cu) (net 15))
 (segment (start 172.085 106.68) (end 172.085 104.14) (width 0.25) (layer F.Cu) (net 15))
 (segment (start 172.085 104.14) (end 170.815 102.87) (width 0.25) (layer F.Cu) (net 15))
 (segment (start 173.355 109.22) (end 173.355 107.95) (width 0.25) (layer F.Cu) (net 14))
 (segment (start 173.355 107.95) (end 174.625 106.68) (width 0.25) (layer F.Cu) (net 14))
 (segment (start 174.625 106.68) (end 174.625 104.14) (width 0.25) (layer F.Cu) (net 14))
 (segment (start 174.625 104.14) (end 173.355 102.87) (width 0.25) (layer F.Cu) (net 14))
 (segment (start 175.895 109.22) (end 175.895 107.95) (width 0.25) (layer F.Cu) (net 13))
 (segment (start 175.895 107.95) (end 177.165 106.68) (width 0.25) (layer F.Cu) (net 13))
 (segment (start 177.165 106.68) (end 177.165 104.14) (width 0.25) (layer F.Cu) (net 13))
 (segment (start 177.165 104.14) (end 175.895 102.87) (width 0.25) (layer F.Cu) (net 13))
 (segment (start 178.435 109.22) (end 178.435 107.95) (width 0.25) (layer F.Cu) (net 12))
 (segment (start 178.435 107.95) (end 179.705 106.68) (width 0.25) (layer F.Cu) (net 12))
 (segment (start 179.705 106.68) (end 179.705 104.14) (width 0.25) (layer F.Cu) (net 12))
 (segment (start 179.705 104.14) (end 178.435 102.87) (width 0.25) (layer F.Cu) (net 12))
 (segment (start 180.975 109.22) (end 180.975 107.95) (width 0.25) (layer F.Cu) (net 11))
 (segment (start 180.975 107.95) (end 182.245 106.68) (width 0.25) (layer F.Cu) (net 11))
 (segment (start 182.245 106.68) (end 182.245 104.14) (width 0.25) (layer F.Cu) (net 11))
 (segment (start 182.245 104.14) (end 180.975 102.87) (width 0.25) (layer F.Cu) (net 11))
 (segment (start 183.515 109.22) (end 183.515 107.95) (width 0.25) (layer F.Cu) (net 7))
 (segment (start 183.515 107.95) (end 184.785 106.68) (width 0.25) (layer F.Cu) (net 7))
 (segment (start 184.785 106.68) (end 184.785 104.14) (width 0.25) (layer F.Cu) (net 7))
 (segment (start 184.785 104.14) (end 183.515 102.87) (width 0.25) (layer F.Cu) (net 7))
 (segment (start 183.515 100.965) (end 182.235654 99.685654) (width 0.25) (layer F.Cu) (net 7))
 (segment (start 183.515 102.87) (end 183.515 100.965) (width 0.25) (layer F.Cu) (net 7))
 (segment (start 187.325 104.14) (end 186.055 102.87) (width 0.25) (layer F.Cu) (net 8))
 (segment (start 187.325 106.68) (end 187.325 104.14) (width 0.25) (layer F.Cu) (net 8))
 (segment (start 186.055 107.95) (end 187.325 106.68) (width 0.25) (layer F.Cu) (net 8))
 (segment (start 186.055 109.22) (end 186.055 107.95) (width 0.25) (layer F.Cu) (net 8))
 (segment (start 186.055 102.87) (end 186.055 99.695) (width 0.25) (layer F.Cu) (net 8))
 (segment (start 188.595 109.22) (end 188.595 107.95) (width 0.25) (layer F.Cu) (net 9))
 (segment (start 188.595 107.95) (end 189.865 106.68) (width 0.25) (layer F.Cu) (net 9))
 (segment (start 189.865 106.68) (end 189.865 104.14) (width 0.25) (layer F.Cu) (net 9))
 (segment (start 189.865 104.14) (end 188.595 102.87) (width 0.25) (layer F.Cu) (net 9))
 (segment (start 188.595 100.946308) (end 189.855654 99.685654) (width 0.25) (layer F.Cu) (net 9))
 (segment (start 188.595 102.87) (end 188.595 100.946308) (width 0.25) (layer F.Cu) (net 9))
 (segment (start 191.135 109.22) (end 191.135 107.95) (width 0.25) (layer F.Cu) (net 10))
 (segment (start 191.135 107.95) (end 192.405 106.68) (width 0.25) (layer F.Cu) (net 10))
 (segment (start 192.405 106.68) (end 192.405 104.14) (width 0.25) (layer F.Cu) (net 10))
 (segment (start 192.405 104.14) (end 191.135 102.87) (width 0.25) (layer F.Cu) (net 10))
 (segment (start 193.675 109.22) (end 193.675 107.95) (width 0.25) (layer F.Cu) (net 4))
 (segment (start 193.675 107.95) (end 194.945 106.68) (width 0.25) (layer F.Cu) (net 4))
 (segment (start 194.945 106.68) (end 194.945 104.14) (width 0.25) (layer F.Cu) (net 4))
 (segment (start 194.945 104.14) (end 193.675 102.87) (width 0.25) (layer F.Cu) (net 4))
 (segment (start 193.675 102.87) (end 193.675 99.695) (width 0.25) (layer F.Cu) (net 4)))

